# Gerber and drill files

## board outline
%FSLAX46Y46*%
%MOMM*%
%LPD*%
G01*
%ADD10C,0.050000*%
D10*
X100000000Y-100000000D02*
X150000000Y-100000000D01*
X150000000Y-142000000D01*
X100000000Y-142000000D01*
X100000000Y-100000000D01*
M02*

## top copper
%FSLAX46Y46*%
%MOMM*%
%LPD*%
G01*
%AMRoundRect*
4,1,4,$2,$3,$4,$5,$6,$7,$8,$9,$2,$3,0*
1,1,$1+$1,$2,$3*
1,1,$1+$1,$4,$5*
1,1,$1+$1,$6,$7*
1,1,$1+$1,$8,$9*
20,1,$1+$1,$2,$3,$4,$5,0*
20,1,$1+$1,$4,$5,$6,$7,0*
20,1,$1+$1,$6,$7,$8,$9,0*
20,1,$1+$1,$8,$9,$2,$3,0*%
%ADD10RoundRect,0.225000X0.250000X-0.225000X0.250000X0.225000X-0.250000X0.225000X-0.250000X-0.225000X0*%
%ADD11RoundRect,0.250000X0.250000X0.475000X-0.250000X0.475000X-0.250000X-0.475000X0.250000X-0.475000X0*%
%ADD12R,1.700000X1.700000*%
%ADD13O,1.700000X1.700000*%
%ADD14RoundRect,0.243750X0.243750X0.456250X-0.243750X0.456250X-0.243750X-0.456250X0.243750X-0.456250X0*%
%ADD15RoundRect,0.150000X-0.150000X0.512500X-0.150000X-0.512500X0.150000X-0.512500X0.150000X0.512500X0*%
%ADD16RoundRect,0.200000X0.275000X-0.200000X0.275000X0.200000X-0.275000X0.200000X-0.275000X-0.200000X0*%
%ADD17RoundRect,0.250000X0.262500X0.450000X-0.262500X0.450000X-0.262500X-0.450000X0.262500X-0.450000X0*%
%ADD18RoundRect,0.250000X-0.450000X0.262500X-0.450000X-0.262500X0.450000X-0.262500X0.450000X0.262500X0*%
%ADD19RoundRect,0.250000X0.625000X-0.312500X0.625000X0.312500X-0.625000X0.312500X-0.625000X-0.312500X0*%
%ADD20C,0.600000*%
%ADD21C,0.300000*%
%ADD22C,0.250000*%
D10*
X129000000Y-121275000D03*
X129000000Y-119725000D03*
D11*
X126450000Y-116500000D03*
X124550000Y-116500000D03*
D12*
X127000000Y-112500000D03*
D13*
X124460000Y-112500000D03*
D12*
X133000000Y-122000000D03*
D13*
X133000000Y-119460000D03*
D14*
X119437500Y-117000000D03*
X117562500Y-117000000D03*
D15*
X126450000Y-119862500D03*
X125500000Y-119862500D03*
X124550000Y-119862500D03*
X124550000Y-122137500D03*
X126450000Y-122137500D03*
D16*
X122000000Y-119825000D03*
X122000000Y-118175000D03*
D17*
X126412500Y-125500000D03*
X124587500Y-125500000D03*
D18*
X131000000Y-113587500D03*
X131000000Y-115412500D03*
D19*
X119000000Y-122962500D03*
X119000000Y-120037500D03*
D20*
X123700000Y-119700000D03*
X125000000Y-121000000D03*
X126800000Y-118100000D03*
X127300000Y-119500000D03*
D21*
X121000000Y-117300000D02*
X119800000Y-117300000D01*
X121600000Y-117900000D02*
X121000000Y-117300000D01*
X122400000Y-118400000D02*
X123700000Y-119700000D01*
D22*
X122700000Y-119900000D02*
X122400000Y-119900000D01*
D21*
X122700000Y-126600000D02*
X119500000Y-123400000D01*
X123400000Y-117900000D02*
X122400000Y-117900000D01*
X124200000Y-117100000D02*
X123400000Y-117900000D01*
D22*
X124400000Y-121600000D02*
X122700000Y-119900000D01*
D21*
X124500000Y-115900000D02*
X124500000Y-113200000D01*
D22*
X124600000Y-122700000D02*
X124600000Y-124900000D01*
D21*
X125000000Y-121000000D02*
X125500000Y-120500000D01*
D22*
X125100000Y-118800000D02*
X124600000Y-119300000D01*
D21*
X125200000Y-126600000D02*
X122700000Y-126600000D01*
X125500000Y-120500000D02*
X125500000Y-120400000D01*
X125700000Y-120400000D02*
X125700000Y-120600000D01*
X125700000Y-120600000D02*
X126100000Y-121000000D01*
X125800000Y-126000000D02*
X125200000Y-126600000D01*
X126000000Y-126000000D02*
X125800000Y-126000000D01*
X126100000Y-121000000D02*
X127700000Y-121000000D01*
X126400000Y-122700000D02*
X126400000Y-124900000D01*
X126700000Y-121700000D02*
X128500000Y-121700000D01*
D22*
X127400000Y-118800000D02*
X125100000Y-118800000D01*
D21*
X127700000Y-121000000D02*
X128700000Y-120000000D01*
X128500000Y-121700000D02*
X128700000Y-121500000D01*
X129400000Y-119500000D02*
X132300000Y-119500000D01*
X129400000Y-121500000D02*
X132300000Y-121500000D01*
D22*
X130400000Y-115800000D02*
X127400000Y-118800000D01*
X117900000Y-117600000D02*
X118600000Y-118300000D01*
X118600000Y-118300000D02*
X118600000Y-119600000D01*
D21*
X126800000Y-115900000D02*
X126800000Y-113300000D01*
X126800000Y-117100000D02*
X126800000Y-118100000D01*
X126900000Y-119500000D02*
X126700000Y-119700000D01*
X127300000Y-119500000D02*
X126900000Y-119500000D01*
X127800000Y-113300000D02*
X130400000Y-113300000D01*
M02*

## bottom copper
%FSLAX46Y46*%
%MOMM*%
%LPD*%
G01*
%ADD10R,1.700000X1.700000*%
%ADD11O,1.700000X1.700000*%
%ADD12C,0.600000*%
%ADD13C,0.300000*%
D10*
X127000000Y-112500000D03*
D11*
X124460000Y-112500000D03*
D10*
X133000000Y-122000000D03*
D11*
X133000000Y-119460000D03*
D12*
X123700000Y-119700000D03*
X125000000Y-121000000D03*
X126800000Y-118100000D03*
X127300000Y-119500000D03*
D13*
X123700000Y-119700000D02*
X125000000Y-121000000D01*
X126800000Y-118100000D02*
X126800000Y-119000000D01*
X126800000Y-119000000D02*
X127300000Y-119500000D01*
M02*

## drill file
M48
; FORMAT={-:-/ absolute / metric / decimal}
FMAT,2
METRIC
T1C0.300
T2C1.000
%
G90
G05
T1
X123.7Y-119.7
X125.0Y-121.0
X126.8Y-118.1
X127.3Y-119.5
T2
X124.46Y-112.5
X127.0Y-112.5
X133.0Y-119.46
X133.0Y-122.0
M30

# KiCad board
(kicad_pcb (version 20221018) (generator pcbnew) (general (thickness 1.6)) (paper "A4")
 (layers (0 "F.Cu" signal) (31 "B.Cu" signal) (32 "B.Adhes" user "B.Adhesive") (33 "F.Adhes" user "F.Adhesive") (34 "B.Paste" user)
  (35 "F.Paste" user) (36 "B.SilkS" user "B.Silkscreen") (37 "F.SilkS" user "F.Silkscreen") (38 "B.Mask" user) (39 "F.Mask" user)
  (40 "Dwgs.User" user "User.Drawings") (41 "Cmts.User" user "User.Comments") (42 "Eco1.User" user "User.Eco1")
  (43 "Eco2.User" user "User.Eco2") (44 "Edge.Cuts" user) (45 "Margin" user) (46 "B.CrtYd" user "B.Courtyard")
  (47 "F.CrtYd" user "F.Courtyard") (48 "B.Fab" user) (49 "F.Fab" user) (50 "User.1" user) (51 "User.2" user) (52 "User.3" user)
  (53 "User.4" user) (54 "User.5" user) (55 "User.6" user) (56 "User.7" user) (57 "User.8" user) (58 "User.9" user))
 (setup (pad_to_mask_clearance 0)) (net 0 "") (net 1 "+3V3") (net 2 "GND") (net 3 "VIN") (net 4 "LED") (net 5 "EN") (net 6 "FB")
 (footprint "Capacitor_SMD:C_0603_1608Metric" (layer "F.Cu") (at 129 120.5 90)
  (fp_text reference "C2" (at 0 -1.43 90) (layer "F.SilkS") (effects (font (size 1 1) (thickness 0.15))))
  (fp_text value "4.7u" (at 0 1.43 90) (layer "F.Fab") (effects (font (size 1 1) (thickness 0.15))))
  (pad "1" smd roundrect (at -0.775 0 90) (size 0.9 0.95) (layers "F.Cu" "F.Paste" "F.Mask") (roundrect_rratio 0.25) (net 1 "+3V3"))
  (pad "2" smd roundrect (at 0.775 0 90) (size 0.9 0.95) (layers "F.Cu" "F.Paste" "F.Mask") (roundrect_rratio 0.25) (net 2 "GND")))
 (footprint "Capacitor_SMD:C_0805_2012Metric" (layer "F.Cu") (at 125.5 116.5 180)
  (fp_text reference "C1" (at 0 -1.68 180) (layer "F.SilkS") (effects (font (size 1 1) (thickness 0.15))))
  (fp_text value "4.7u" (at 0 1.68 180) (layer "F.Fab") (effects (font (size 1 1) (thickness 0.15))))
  (pad "1" smd roundrect (at -0.95 0 180) (size 1 1.45) (layers "F.Cu" "F.Paste" "F.Mask") (roundrect_rratio 0.25) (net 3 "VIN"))
  (pad "2" smd roundrect (at 0.95 0 180) (size 1 1.45) (layers "F.Cu" "F.Paste" "F.Mask") (roundrect_rratio 0.25) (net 2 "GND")))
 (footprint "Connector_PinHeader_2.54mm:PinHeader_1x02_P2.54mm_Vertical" (layer "F.Cu") (at 127 112.5 -90)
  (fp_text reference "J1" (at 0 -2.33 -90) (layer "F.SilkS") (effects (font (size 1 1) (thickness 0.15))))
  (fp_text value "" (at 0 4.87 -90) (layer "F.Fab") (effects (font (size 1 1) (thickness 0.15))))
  (pad "1" thru_hole rect (at 0 0 270) (size 1.7 1.7) (drill 1) (layers "*.Cu" "*.Mask") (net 3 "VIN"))
  (pad "2" thru_hole oval (at 0 2.54 270) (size 1.7 1.7) (drill 1) (layers "*.Cu" "*.Mask") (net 2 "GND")))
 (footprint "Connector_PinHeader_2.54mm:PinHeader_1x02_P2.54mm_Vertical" (layer "F.Cu") (at 133 122 180)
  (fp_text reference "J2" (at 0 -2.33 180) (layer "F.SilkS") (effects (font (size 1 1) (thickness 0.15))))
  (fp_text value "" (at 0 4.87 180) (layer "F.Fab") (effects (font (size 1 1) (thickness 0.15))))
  (pad "1" thru_hole rect (at 0 0 180) (size 1.7 1.7) (drill 1) (layers "*.Cu" "*.Mask") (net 1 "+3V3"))
  (pad "2" thru_hole oval (at 0 2.54 180) (size 1.7 1.7) (drill 1) (layers "*.Cu" "*.Mask") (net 2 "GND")))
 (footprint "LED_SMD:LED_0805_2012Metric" (layer "F.Cu") (at 118.5 117 180)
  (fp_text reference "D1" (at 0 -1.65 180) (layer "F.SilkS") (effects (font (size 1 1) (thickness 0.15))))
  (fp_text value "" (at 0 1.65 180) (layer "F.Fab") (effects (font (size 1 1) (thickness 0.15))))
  (pad "1" smd roundrect (at -0.9375 0 180) (size 0.975 1.4) (layers "F.Cu" "F.Paste" "F.Mask") (roundrect_rratio 0.25) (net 2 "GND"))
  (pad "2" smd roundrect (at 0.9375 0 180) (size 0.975 1.4) (layers "F.Cu" "F.Paste" "F.Mask") (roundrect_rratio 0.25) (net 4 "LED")))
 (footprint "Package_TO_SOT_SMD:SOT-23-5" (layer "F.Cu") (at 125.5 121 -90)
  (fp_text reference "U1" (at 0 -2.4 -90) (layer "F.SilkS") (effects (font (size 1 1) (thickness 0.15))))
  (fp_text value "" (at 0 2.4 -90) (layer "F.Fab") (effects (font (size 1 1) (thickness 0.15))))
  (pad "1" smd roundrect (at -1.1375 -0.95 270) (size 1.325 0.6) (layers "F.Cu" "F.Paste" "F.Mask") (roundrect_rratio 0.25) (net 3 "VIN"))
  (pad "2" smd roundrect (at -1.1375 0 270) (size 1.325 0.6) (layers "F.Cu" "F.Paste" "F.Mask") (roundrect_rratio 0.25) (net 2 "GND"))
  (pad "3" smd roundrect (at -1.1375 0.95 270) (size 1.325 0.6) (layers "F.Cu" "F.Paste" "F.Mask") (roundrect_rratio 0.25) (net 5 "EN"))
  (pad "4" smd roundrect (at 1.1375 0.95 270) (size 1.325 0.6) (layers "F.Cu" "F.Paste" "F.Mask") (roundrect_rratio 0.25) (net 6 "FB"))
  (pad "5" smd roundrect (at 1.1375 -0.95 270) (size 1.325 0.6) (layers "F.Cu" "F.Paste" "F.Mask") (roundrect_rratio 0.25) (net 1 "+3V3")))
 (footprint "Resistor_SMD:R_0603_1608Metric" (layer "F.Cu") (at 122 119 90)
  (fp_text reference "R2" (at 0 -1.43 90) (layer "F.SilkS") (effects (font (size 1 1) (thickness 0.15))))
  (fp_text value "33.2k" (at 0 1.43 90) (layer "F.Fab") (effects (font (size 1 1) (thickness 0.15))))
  (pad "1" smd roundrect (at -0.825 0 90) (size 0.8 0.95) (layers "F.Cu" "F.Paste" "F.Mask") (roundrect_rratio 0.25) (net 6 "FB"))
  (pad "2" smd roundrect (at 0.825 0 90) (size 0.8 0.95) (layers "F.Cu" "F.Paste" "F.Mask") (roundrect_rratio 0.25) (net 2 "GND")))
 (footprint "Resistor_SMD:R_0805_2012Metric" (layer "F.Cu") (at 125.5 125.5 180)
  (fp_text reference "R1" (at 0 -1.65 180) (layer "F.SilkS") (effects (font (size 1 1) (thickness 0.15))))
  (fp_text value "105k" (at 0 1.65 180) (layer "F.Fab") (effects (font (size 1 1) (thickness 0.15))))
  (pad "1" smd roundrect (at -0.9125 0 180) (size 1.025 1.4) (layers "F.Cu" "F.Paste" "F.Mask") (roundrect_rratio 0.243902) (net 1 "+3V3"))
  (pad "2" smd roundrect (at 0.9125 0 180) (size 1.025 1.4) (layers "F.Cu" "F.Paste" "F.Mask") (roundrect_rratio 0.243902) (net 6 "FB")))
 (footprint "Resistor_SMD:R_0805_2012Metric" (layer "F.Cu") (at 131 114.5 -90)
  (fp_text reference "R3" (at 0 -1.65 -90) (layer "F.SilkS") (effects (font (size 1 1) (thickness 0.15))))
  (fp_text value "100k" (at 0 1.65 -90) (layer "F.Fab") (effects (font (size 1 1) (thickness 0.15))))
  (pad "1" smd roundrect (at -0.9125 0 270) (size 1.025 1.4) (layers "F.Cu" "F.Paste" "F.Mask") (roundrect_rratio 0.243902) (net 3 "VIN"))
  (pad "2" smd roundrect (at 0.9125 0 270) (size 1.025 1.4) (layers "F.Cu" "F.Paste" "F.Mask") (roundrect_rratio 0.243902) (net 5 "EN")))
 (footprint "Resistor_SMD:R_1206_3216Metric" (layer "F.Cu") (at 119 121.5 90)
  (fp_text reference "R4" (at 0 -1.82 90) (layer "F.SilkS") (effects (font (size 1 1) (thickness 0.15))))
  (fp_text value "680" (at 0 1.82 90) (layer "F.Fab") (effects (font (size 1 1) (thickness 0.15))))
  (pad "1" smd roundrect (at -1.4625 0 90) (size 1.125 1.75) (layers "F.Cu" "F.Paste" "F.Mask") (roundrect_rratio 0.222222) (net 1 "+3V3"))
  (pad "2" smd roundrect (at 1.4625 0 90) (size 1.125 1.75) (layers "F.Cu" "F.Paste" "F.Mask") (roundrect_rratio 0.222222) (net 4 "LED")))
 (gr_rect (start 100 100) (end 150 142) (stroke (width 0.05) (type default)) (fill none) (layer "Edge.Cuts"))
 (segment (start 121 117.3) (end 119.8 117.3) (width 0.3) (layer "F.Cu") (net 2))
 (segment (start 121.6 117.9) (end 121 117.3) (width 0.3) (layer "F.Cu") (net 2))
 (segment (start 122.4 118.4) (end 123.7 119.7) (width 0.3) (layer "F.Cu") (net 2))
 (segment (start 122.7 119.9) (end 122.4 119.9) (width 0.25) (layer "F.Cu") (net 6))
 (segment (start 122.7 126.6) (end 119.5 123.4) (width 0.3) (layer "F.Cu") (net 1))
 (segment (start 123.4 117.9) (end 122.4 117.9) (width 0.3) (layer "F.Cu") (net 2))
 (segment (start 124.2 117.1) (end 123.4 117.9) (width 0.3) (layer "F.Cu") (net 2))
 (segment (start 124.4 121.6) (end 122.7 119.9) (width 0.25) (layer "F.Cu") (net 6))
 (segment (start 124.5 115.9) (end 124.5 113.2) (width 0.3) (layer "F.Cu") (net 2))
 (segment (start 124.6 122.7) (end 124.6 124.9) (width 0.25) (layer "F.Cu") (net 6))
 (segment (start 125 121) (end 125.5 120.5) (width 0.3) (layer "F.Cu") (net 2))
 (segment (start 125.1 118.8) (end 124.6 119.3) (width 0.25) (layer "F.Cu") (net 5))
 (segment (start 125.2 126.6) (end 122.7 126.6) (width 0.3) (layer "F.Cu") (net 1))
 (segment (start 125.5 120.5) (end 125.5 120.4) (width 0.3) (layer "F.Cu") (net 2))
 (segment (start 125.7 120.4) (end 125.7 120.6) (width 0.3) (layer "F.Cu") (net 2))
 (segment (start 125.7 120.6) (end 126.1 121) (width 0.3) (layer "F.Cu") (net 2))
 (segment (start 125.8 126) (end 125.2 126.6) (width 0.3) (layer "F.Cu") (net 1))
 (segment (start 126 126) (end 125.8 126) (width 0.3) (layer "F.Cu") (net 1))
 (segment (start 126.1 121) (end 127.7 121) (width 0.3) (layer "F.Cu") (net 2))
 (segment (start 126.4 122.7) (end 126.4 124.9) (width 0.3) (layer "F.Cu") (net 1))
 (segment (start 126.7 121.7) (end 128.5 121.7) (width 0.3) (layer "F.Cu") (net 1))
 (segment (start 127.4 118.8) (end 125.1 118.8) (width 0.25) (layer "F.Cu") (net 5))
 (segment (start 127.7 121) (end 128.7 120) (width 0.3) (layer "F.Cu") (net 2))
 (segment (start 128.5 121.7) (end 128.7 121.5) (width 0.3) (layer "F.Cu") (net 1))
 (segment (start 129.4 119.5) (end 132.3 119.5) (width 0.3) (layer "F.Cu") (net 2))
 (segment (start 129.4 121.5) (end 132.3 121.5) (width 0.3) (layer "F.Cu") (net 1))
 (segment (start 130.4 115.8) (end 127.4 118.8) (width 0.25) (layer "F.Cu") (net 5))
 (via (at 123.7 119.7) (size 0.6) (drill 0.3) (layers "F.Cu" "B.Cu") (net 2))
 (via (at 125 121) (size 0.6) (drill 0.3) (layers "F.Cu" "B.Cu") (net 2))
 (segment (start 117.9 117.6) (end 118.6 118.3) (width 0.25) (layer "F.Cu") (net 4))
 (segment (start 118.6 118.3) (end 118.6 119.6) (width 0.25) (layer "F.Cu") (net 4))
 (segment (start 123.7 119.7) (end 125 121) (width 0.3) (layer "B.Cu") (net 2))
 (segment (start 126.8 115.9) (end 126.8 113.3) (width 0.3) (layer "F.Cu") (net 3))
 (segment (start 126.8 117.1) (end 126.8 118.1) (width 0.3) (layer "F.Cu") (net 3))
 (segment (start 126.9 119.5) (end 126.7 119.7) (width 0.3) (layer "F.Cu") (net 3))
 (segment (start 127.3 119.5) (end 126.9 119.5) (width 0.3) (layer "F.Cu") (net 3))
 (segment (start 127.8 113.3) (end 130.4 113.3) (width 0.3) (layer "F.Cu") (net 3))
 (via (at 126.8 118.1) (size 0.6) (drill 0.3) (layers "F.Cu" "B.Cu") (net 3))
 (via (at 127.3 119.5) (size 0.6) (drill 0.3) (layers "F.Cu" "B.Cu") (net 3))
 (segment (start 126.8 118.1) (end 126.8 119) (width 0.3) (layer "B.Cu") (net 3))
 (segment (start 126.8 119) (end 127.3 119.5) (width 0.3) (layer "B.Cu") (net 3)))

